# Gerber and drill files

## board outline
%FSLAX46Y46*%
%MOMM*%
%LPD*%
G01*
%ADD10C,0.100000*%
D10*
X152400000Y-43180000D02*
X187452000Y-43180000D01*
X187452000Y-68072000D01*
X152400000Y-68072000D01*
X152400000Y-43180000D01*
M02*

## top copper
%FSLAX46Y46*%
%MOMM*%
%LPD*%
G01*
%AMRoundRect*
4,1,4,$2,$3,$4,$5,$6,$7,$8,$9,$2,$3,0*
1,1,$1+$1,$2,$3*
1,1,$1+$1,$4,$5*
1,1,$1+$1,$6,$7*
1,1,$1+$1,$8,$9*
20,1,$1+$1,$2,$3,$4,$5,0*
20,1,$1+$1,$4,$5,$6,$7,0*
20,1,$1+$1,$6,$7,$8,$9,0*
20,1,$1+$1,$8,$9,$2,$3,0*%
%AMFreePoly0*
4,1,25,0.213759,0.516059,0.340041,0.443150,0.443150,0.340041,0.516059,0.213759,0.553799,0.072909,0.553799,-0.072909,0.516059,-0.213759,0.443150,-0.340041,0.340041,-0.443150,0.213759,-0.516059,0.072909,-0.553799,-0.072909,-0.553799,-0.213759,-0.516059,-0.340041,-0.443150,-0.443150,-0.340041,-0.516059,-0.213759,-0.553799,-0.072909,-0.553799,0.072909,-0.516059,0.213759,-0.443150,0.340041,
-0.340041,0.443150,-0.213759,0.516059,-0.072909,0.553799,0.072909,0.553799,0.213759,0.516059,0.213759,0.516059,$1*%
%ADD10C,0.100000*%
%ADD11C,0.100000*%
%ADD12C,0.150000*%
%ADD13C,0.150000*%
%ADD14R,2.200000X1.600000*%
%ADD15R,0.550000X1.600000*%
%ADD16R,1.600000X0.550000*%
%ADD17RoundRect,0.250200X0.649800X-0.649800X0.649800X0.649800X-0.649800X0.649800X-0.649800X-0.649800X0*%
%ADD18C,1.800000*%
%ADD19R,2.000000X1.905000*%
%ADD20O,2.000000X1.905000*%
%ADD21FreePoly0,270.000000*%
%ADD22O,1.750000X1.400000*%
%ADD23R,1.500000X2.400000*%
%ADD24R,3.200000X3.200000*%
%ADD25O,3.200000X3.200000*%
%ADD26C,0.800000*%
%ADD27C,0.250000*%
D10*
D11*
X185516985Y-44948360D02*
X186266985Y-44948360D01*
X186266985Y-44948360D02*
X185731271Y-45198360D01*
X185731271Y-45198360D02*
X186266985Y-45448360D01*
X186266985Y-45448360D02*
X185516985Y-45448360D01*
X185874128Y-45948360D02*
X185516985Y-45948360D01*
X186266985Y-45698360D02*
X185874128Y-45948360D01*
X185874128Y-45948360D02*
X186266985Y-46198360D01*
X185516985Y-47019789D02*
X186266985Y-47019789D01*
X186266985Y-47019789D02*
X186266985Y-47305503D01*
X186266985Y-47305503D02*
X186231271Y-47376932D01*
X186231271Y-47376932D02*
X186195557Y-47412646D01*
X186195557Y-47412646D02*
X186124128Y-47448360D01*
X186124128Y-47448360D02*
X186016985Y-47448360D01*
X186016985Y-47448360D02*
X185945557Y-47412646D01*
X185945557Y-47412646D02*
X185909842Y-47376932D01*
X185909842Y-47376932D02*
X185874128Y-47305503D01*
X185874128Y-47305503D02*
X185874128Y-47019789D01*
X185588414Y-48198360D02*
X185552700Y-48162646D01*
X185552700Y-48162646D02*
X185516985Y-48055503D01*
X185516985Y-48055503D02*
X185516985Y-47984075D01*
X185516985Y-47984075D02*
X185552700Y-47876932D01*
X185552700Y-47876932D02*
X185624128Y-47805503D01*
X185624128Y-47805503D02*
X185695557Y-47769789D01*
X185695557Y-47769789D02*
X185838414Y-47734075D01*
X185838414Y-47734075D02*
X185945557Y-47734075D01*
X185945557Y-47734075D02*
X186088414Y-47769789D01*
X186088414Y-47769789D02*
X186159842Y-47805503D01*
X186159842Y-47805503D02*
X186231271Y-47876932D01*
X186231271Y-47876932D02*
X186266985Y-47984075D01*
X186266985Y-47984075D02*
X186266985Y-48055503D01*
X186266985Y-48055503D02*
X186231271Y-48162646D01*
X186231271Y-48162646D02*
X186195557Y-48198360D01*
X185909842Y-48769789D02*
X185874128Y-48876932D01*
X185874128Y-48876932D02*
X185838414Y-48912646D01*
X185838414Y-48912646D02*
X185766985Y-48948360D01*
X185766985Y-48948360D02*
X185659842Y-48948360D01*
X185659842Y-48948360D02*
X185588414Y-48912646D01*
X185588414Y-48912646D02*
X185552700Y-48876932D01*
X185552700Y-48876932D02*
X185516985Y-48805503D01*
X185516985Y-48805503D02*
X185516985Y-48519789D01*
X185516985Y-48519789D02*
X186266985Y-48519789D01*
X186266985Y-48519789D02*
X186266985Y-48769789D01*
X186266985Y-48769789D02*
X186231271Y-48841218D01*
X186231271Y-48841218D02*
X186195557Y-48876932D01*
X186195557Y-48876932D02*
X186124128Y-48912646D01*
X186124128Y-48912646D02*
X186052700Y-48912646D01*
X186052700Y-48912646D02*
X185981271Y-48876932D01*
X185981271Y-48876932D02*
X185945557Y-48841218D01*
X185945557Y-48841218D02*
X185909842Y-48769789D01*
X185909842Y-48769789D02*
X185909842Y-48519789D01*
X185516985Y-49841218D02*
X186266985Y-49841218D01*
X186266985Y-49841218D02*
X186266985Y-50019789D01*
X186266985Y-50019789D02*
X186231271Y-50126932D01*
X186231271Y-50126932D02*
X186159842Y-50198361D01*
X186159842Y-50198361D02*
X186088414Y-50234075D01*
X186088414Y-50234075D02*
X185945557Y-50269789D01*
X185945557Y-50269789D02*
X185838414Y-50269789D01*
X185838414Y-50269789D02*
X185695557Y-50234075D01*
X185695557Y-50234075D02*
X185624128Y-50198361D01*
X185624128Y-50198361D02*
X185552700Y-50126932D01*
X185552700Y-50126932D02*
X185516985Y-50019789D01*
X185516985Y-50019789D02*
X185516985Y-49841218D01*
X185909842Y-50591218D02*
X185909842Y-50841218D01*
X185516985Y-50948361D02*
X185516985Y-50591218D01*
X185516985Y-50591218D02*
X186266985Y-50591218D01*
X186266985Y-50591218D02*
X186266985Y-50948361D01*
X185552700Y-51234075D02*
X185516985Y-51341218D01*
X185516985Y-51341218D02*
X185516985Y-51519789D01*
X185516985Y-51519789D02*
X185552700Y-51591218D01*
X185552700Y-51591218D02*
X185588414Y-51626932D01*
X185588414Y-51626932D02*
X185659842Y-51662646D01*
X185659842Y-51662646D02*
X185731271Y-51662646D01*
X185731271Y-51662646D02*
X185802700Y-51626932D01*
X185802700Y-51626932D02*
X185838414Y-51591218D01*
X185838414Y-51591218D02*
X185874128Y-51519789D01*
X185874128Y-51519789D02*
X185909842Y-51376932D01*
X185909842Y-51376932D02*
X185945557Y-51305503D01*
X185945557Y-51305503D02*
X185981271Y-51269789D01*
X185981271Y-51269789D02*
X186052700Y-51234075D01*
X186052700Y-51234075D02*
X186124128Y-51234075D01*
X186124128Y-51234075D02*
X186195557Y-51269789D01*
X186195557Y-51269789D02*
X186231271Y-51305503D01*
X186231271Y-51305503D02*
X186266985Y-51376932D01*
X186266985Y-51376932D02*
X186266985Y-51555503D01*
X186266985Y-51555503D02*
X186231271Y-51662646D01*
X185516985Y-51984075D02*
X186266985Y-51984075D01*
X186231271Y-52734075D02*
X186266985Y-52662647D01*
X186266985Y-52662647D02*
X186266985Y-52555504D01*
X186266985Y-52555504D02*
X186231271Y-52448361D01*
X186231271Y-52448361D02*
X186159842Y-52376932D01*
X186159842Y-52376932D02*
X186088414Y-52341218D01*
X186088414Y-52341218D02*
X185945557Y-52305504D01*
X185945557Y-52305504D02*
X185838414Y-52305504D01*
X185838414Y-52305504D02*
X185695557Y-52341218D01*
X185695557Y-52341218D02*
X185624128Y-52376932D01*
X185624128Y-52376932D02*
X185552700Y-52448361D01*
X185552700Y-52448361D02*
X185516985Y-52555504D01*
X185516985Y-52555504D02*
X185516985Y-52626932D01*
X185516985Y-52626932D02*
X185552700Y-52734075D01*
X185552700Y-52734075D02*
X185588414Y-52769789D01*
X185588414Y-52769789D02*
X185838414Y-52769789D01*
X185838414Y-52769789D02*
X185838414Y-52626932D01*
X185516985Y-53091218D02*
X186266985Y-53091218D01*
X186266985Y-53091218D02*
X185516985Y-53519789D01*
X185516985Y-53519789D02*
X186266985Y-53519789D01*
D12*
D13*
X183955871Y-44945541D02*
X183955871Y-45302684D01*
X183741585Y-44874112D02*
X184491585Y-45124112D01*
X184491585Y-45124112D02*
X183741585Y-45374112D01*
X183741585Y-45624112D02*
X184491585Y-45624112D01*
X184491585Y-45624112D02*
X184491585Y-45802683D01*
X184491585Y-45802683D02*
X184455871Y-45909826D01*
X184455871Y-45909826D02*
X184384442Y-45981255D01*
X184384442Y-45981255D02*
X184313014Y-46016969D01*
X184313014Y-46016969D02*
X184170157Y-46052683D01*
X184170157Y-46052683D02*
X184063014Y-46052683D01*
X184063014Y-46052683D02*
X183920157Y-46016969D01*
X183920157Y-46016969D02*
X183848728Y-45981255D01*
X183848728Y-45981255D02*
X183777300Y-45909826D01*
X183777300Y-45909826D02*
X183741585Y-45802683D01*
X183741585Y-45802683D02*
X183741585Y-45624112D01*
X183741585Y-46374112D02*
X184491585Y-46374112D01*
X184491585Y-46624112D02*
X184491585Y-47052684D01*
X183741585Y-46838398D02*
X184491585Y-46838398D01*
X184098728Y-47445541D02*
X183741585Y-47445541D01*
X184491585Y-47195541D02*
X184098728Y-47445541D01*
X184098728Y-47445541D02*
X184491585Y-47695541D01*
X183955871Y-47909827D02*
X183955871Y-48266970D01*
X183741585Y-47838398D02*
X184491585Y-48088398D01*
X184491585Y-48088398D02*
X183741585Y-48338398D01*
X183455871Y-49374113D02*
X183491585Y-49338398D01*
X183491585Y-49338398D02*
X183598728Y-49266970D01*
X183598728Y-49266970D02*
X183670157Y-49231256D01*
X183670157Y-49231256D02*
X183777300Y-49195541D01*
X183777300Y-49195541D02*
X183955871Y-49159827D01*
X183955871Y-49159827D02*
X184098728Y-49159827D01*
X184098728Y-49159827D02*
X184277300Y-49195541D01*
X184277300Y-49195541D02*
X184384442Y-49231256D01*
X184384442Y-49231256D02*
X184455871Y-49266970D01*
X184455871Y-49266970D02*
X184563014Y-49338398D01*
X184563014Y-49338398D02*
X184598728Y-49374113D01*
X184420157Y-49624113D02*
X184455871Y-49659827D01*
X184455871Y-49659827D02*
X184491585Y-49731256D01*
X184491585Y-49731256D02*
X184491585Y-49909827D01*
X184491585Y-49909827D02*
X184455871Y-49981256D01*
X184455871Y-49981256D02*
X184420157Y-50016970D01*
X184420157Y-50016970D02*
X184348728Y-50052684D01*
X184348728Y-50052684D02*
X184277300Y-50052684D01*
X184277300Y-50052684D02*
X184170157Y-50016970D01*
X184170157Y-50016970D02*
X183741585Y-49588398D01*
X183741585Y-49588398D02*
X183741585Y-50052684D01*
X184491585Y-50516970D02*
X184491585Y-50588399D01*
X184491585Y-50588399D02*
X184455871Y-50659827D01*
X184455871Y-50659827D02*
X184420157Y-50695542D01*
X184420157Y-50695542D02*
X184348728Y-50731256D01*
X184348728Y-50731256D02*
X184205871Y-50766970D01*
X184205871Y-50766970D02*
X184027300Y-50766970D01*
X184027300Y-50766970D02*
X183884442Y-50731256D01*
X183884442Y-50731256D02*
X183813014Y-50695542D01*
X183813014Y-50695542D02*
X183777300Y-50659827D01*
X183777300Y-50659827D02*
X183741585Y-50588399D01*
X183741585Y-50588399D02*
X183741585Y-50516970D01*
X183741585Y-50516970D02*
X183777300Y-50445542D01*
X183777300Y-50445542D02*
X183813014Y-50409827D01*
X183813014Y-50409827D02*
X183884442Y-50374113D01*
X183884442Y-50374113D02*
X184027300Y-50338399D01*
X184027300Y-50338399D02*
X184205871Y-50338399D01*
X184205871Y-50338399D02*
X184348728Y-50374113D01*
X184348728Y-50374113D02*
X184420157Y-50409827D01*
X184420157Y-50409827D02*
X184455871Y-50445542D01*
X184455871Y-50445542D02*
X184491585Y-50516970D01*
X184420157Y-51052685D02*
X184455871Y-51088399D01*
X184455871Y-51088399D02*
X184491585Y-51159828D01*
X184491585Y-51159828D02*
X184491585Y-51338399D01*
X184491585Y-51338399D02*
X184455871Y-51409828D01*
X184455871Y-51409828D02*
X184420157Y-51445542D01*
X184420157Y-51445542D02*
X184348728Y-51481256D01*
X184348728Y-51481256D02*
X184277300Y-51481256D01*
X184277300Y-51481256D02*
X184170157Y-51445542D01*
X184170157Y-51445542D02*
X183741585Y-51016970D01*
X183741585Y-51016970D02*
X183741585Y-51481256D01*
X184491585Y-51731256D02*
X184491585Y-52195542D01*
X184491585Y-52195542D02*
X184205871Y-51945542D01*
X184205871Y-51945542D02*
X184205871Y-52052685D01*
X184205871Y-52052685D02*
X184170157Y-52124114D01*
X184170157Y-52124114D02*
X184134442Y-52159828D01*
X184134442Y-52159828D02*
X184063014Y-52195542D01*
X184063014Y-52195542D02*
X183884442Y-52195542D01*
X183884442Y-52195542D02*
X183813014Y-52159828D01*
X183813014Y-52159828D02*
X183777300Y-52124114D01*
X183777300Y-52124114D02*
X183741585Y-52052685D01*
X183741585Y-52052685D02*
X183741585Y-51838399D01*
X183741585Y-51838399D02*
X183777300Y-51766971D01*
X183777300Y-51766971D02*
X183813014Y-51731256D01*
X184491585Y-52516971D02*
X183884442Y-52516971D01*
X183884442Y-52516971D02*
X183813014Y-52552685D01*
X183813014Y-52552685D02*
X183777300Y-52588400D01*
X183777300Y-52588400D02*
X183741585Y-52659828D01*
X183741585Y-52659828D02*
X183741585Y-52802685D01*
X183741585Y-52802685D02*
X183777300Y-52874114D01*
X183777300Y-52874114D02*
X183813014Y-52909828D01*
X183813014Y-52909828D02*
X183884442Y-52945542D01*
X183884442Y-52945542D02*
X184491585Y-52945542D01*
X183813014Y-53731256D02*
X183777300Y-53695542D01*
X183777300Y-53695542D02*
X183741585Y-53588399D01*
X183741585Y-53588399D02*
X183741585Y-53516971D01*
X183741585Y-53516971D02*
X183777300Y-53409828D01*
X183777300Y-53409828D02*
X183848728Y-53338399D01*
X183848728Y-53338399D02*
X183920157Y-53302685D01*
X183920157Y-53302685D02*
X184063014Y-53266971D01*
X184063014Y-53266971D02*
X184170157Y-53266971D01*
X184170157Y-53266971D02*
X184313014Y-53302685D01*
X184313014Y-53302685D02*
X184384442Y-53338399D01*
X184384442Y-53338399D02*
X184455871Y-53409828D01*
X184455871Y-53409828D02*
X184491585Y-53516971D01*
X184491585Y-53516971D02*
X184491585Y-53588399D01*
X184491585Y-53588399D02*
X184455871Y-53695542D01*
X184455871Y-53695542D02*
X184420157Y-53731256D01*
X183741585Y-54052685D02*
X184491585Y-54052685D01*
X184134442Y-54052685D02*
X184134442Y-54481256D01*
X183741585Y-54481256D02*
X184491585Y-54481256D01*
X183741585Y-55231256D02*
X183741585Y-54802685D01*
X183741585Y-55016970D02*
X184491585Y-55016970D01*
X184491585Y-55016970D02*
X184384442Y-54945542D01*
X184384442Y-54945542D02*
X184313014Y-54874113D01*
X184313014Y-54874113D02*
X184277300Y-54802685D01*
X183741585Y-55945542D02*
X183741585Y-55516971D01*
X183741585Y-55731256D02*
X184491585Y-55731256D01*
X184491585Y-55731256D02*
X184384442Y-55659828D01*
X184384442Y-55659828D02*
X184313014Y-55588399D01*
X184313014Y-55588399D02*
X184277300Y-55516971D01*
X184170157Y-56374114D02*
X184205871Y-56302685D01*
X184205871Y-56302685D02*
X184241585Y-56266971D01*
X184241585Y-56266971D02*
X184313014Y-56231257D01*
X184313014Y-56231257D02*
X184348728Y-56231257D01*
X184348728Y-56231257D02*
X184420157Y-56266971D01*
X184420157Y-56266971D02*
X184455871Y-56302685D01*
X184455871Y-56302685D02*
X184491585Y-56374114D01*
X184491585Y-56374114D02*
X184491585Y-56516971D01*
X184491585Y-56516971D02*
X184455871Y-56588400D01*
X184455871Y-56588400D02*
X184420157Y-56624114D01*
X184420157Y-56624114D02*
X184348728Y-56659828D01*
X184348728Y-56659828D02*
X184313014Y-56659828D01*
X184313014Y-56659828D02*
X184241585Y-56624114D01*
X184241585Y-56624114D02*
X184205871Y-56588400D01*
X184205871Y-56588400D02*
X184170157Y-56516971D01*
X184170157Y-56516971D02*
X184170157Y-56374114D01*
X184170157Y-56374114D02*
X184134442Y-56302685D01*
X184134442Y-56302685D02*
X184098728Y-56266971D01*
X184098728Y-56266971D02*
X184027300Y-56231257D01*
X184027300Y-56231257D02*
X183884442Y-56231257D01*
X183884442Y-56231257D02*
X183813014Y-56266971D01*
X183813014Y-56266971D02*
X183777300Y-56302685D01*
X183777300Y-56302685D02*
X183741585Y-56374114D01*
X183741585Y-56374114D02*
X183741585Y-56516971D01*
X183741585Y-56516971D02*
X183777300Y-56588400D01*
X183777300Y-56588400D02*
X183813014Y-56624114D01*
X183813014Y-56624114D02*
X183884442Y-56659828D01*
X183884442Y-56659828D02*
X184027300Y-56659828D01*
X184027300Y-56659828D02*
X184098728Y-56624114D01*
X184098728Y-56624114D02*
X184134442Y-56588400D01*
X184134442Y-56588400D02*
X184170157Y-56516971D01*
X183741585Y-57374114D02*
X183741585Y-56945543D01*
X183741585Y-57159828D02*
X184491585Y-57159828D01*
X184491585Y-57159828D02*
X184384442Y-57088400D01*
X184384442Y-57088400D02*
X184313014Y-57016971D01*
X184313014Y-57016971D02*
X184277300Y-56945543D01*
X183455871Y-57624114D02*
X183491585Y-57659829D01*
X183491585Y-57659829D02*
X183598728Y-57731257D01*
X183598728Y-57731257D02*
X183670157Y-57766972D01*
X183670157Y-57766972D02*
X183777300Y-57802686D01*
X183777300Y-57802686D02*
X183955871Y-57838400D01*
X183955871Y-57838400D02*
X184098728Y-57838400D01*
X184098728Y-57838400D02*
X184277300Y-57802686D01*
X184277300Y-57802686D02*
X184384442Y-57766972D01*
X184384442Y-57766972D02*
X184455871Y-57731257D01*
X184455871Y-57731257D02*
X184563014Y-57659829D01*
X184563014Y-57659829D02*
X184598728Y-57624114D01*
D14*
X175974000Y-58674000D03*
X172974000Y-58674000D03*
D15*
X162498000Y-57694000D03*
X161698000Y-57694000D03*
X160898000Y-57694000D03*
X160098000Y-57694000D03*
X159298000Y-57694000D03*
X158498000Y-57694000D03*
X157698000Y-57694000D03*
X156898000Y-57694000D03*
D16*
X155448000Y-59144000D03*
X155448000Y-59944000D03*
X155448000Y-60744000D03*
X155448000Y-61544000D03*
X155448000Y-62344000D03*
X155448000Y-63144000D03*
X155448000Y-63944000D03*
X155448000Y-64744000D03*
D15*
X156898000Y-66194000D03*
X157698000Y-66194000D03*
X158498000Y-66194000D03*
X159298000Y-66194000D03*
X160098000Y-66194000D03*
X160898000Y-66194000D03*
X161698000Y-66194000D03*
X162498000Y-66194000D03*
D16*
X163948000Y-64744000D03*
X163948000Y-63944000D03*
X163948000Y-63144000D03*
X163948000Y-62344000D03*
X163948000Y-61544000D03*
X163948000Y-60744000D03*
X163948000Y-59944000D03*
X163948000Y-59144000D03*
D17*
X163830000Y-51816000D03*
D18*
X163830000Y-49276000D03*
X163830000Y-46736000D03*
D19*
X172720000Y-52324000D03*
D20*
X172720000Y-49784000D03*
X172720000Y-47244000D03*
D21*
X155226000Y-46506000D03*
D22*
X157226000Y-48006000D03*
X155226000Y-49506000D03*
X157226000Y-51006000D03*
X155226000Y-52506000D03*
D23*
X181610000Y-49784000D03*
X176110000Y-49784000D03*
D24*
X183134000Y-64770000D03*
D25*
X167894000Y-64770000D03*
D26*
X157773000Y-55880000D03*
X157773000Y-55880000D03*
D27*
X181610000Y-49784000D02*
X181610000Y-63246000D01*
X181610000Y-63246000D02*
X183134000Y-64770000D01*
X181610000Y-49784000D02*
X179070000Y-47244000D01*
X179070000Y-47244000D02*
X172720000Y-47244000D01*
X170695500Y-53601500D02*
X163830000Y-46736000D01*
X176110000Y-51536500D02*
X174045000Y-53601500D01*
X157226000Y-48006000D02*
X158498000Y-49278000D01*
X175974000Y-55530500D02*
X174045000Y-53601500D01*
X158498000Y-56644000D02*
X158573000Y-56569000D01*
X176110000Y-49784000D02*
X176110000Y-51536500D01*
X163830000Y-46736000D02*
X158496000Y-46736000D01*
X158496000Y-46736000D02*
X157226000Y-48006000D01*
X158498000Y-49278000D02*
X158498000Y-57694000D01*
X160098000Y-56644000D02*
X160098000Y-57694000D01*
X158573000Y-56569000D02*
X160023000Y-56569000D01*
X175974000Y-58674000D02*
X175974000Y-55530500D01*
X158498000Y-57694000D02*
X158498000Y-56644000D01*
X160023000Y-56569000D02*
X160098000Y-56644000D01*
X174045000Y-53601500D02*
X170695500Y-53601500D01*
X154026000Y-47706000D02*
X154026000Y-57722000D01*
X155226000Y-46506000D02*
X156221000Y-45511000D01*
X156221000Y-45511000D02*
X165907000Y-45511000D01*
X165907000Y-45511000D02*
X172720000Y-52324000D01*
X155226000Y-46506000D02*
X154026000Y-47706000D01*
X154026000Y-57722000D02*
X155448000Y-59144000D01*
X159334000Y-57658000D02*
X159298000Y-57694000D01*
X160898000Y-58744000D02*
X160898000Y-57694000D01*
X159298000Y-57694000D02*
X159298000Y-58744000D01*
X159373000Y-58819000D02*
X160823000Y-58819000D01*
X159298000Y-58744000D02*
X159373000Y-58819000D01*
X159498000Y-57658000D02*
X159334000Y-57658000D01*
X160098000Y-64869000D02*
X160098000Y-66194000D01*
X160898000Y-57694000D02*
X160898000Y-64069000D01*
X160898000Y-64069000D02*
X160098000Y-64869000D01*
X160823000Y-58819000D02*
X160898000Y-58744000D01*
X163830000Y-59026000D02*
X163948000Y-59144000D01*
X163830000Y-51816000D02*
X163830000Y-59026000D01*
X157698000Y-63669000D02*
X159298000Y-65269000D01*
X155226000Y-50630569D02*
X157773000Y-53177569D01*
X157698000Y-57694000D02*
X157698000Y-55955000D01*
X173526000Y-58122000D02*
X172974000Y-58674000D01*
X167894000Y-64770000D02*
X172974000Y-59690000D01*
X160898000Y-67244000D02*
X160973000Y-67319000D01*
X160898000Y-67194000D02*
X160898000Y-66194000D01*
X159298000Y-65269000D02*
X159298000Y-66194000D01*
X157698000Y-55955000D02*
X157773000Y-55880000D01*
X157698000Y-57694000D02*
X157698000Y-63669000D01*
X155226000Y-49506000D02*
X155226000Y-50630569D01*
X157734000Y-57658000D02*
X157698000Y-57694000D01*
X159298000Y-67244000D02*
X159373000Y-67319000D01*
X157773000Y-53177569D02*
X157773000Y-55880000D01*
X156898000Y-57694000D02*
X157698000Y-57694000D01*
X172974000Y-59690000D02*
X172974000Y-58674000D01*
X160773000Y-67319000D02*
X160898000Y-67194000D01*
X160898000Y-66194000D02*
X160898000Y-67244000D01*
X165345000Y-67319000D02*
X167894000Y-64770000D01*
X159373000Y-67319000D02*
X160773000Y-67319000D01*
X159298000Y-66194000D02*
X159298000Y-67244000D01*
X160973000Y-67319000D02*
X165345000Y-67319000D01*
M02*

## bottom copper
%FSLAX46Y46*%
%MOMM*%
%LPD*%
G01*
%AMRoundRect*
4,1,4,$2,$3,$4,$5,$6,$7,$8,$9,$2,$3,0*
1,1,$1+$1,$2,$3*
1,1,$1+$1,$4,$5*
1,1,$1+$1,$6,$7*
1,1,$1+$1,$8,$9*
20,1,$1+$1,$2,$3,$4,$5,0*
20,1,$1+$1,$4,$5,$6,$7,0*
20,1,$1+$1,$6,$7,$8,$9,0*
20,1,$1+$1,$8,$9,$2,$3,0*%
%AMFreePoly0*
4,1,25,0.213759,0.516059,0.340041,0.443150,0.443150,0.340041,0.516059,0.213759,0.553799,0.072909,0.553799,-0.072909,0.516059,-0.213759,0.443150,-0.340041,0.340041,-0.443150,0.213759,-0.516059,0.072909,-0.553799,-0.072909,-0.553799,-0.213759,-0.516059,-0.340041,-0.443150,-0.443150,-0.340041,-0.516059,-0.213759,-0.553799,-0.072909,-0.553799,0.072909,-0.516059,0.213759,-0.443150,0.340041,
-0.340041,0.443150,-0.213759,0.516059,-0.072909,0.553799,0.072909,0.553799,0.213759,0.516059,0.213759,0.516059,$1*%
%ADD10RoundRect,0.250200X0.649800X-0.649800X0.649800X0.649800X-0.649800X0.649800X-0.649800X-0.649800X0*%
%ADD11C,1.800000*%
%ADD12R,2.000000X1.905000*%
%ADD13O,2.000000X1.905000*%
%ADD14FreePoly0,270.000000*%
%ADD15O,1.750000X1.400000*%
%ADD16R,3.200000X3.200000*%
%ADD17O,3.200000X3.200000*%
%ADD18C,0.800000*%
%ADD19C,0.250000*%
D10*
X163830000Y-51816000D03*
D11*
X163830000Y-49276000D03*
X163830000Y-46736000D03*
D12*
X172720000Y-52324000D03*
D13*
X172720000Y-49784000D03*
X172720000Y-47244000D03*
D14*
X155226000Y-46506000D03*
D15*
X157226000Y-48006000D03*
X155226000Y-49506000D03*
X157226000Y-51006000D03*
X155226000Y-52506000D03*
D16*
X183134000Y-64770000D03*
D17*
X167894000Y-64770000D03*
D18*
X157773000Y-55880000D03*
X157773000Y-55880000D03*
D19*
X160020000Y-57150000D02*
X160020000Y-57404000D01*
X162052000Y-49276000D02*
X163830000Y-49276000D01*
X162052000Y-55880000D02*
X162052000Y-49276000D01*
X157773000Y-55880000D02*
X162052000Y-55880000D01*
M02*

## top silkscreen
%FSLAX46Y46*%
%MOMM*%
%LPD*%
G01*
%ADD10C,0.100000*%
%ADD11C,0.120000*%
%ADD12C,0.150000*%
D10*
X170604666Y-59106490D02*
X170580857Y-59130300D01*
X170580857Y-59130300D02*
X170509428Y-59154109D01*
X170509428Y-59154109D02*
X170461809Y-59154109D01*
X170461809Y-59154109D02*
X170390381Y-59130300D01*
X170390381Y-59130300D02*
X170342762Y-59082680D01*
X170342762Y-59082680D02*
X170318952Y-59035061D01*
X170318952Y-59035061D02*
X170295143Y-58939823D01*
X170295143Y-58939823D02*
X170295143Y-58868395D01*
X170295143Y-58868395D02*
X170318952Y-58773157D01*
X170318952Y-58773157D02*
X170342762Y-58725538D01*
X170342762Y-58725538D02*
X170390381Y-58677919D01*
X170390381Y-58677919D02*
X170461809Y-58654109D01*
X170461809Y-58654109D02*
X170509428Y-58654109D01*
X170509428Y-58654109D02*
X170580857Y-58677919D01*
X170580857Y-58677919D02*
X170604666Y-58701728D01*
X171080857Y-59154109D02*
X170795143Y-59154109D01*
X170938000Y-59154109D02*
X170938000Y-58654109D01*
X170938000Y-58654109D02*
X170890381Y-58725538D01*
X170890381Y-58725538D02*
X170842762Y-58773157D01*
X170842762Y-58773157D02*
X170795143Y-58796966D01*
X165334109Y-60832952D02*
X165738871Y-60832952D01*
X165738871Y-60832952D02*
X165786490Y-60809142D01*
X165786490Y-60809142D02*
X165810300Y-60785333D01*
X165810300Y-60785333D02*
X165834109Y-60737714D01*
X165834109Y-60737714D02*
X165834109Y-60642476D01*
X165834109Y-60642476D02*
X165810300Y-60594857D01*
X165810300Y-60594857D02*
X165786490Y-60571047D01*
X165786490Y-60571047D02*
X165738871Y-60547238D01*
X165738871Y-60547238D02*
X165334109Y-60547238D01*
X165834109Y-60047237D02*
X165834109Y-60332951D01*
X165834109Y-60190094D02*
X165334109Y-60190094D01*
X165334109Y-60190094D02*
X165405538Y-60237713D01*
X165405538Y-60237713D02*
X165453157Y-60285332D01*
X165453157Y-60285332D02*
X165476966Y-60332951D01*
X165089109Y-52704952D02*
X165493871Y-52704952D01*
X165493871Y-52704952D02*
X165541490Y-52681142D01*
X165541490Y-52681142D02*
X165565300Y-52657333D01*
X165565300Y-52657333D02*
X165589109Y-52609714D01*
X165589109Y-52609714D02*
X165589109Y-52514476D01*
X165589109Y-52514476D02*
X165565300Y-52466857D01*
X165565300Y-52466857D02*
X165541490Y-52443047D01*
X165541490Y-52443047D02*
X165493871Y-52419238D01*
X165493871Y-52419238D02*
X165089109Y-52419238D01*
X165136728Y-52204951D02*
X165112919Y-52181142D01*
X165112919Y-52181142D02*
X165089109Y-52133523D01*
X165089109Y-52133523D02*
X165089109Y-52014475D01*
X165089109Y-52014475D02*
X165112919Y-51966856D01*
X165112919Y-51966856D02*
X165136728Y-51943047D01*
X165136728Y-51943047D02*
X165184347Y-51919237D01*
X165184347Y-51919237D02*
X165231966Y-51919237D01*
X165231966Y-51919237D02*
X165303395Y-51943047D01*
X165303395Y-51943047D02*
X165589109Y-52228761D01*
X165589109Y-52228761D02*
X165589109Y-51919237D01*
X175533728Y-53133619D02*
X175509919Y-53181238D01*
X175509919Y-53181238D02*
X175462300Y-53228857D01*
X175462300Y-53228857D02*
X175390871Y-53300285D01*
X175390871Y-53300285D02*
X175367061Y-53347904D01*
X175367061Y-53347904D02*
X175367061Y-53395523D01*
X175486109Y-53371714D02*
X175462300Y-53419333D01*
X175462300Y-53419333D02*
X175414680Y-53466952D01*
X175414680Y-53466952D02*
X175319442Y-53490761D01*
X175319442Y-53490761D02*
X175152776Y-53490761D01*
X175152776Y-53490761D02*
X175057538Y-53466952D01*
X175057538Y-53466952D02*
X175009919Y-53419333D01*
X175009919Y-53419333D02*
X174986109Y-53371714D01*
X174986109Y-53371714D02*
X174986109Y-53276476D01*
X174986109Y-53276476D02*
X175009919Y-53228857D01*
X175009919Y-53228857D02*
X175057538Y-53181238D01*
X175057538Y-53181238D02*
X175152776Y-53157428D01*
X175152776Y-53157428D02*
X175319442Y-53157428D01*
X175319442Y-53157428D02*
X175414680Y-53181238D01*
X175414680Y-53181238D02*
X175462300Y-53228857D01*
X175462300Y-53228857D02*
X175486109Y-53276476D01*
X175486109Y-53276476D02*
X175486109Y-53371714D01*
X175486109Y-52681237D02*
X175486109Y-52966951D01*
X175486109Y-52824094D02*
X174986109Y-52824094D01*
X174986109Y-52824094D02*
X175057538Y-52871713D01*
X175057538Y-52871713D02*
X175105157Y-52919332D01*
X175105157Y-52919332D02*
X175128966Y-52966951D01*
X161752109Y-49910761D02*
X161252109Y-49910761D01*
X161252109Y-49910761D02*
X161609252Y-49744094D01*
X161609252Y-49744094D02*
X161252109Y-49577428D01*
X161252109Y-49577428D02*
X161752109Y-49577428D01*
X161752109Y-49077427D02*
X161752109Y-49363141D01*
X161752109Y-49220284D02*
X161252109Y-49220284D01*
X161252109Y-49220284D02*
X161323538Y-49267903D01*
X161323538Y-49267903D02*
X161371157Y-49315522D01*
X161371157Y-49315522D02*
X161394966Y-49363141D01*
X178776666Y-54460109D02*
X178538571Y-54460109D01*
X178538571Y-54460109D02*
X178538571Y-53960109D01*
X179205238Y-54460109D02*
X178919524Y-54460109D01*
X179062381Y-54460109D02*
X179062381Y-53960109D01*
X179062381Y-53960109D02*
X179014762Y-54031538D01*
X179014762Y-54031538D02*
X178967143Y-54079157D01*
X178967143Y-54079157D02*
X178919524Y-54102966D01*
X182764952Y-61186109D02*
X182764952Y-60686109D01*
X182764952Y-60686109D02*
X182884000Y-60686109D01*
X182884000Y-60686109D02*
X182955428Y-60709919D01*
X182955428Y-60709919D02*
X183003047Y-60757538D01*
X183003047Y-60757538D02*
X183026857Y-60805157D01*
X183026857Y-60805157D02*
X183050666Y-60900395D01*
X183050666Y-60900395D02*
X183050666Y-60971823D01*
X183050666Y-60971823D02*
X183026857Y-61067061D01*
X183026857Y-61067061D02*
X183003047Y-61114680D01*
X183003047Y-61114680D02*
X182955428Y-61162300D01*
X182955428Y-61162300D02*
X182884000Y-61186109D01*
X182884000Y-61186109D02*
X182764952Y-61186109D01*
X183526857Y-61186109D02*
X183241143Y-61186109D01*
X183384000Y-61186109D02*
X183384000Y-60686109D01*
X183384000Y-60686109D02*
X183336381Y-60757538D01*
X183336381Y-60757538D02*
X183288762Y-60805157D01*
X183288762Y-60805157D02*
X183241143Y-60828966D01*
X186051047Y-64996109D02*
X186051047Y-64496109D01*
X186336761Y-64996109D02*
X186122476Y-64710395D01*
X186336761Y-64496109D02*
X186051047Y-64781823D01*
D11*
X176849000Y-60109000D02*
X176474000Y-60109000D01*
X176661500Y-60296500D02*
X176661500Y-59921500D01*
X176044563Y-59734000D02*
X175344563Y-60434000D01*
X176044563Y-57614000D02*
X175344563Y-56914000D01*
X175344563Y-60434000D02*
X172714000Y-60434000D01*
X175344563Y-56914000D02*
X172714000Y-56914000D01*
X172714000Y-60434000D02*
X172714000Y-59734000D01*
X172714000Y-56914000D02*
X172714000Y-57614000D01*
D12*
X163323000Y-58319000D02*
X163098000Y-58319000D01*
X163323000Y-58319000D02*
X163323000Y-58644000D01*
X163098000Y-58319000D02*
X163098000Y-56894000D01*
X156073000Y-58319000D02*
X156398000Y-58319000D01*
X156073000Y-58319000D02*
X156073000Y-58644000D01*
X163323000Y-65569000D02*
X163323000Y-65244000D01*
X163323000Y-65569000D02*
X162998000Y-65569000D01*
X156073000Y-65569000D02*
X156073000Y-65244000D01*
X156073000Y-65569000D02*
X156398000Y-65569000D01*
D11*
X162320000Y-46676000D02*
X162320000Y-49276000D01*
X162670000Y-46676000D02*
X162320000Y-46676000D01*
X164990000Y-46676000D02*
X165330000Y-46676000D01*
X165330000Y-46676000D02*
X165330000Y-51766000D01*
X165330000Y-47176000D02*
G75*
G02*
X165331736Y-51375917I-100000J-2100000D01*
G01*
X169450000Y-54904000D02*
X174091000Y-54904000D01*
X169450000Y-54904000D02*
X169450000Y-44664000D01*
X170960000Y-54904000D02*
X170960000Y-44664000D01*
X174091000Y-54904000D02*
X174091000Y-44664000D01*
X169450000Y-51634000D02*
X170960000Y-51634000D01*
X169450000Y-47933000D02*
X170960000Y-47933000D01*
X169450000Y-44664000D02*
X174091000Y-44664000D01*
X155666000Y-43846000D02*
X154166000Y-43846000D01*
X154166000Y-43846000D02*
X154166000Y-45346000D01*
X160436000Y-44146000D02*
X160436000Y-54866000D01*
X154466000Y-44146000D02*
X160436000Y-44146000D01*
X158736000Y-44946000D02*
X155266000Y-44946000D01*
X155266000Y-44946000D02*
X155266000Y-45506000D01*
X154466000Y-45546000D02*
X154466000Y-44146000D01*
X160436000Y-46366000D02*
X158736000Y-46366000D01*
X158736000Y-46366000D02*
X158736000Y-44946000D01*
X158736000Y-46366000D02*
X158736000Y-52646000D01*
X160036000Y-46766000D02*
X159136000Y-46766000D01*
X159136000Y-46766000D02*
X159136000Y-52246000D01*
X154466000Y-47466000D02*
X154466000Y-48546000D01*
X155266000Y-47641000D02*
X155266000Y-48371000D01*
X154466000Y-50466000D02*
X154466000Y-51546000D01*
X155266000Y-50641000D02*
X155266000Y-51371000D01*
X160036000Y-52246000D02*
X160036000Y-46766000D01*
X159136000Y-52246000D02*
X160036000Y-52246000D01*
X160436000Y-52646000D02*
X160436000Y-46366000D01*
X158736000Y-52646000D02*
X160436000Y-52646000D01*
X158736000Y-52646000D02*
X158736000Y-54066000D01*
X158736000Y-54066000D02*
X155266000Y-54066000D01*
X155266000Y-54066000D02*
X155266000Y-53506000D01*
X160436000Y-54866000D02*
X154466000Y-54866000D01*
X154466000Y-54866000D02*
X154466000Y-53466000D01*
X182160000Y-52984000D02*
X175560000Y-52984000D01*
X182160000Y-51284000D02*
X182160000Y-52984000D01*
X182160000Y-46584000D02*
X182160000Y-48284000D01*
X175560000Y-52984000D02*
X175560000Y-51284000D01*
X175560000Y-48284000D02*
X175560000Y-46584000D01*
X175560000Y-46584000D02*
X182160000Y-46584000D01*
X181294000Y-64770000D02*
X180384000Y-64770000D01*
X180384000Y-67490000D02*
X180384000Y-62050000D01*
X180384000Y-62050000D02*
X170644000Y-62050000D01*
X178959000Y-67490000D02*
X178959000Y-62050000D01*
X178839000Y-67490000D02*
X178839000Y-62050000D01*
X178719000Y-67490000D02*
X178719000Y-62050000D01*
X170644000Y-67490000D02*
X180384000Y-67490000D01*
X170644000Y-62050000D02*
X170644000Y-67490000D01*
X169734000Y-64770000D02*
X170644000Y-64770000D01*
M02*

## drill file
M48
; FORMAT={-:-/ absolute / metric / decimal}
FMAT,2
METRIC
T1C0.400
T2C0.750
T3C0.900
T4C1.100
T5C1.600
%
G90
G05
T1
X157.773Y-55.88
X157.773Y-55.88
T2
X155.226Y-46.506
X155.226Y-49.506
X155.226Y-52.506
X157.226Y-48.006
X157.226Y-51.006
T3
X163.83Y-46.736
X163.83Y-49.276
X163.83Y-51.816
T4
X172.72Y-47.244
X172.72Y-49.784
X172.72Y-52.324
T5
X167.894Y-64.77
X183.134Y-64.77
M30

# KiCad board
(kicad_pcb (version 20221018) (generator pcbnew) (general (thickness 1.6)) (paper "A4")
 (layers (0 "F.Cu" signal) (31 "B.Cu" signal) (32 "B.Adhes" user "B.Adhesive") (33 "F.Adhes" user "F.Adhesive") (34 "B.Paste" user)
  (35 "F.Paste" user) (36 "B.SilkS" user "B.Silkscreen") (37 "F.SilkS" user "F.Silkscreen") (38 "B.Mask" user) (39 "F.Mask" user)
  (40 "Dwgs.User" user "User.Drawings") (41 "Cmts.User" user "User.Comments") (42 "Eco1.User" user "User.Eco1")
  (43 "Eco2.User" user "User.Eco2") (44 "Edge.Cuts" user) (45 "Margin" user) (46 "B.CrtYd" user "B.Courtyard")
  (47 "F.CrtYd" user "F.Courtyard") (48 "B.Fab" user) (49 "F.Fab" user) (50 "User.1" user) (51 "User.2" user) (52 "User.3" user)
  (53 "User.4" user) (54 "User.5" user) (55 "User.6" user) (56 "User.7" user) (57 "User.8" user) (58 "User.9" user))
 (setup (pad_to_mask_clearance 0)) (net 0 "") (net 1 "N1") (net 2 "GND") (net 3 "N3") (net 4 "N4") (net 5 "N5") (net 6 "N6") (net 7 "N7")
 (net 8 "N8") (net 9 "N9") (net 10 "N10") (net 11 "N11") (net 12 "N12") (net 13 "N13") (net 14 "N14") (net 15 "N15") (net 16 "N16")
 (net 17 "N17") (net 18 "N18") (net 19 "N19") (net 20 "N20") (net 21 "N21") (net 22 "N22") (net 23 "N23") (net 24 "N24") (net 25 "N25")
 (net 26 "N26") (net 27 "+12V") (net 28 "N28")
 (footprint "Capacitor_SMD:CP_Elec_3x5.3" (layer "F.Cu") (at 174.474 58.674 180)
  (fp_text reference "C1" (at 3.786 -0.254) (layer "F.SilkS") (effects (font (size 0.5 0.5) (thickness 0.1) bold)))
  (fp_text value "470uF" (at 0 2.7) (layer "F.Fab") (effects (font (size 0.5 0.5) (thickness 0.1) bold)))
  (fp_line (start -2.375 -1.435) (end -2 -1.435) (stroke (width 0.12) (type solid)) (layer "F.SilkS"))
  (fp_line (start -2.1875 -1.6225) (end -2.1875 -1.2475) (stroke (width 0.12) (type solid)) (layer "F.SilkS"))
  (fp_line (start -1.570563 -1.06) (end -0.870563 -1.76) (stroke (width 0.12) (type solid)) (layer "F.SilkS"))
  (fp_line (start -1.570563 1.06) (end -0.870563 1.76) (stroke (width 0.12) (type solid)) (layer "F.SilkS"))
  (fp_line (start -0.870563 -1.76) (end 1.76 -1.76) (stroke (width 0.12) (type solid)) (layer "F.SilkS"))
  (fp_line (start -0.870563 1.76) (end 1.76 1.76) (stroke (width 0.12) (type solid)) (layer "F.SilkS"))
  (fp_line (start 1.76 -1.76) (end 1.76 -1.06) (stroke (width 0.12) (type solid)) (layer "F.SilkS"))
  (fp_line (start 1.76 1.76) (end 1.76 1.06) (stroke (width 0.12) (type solid)) (layer "F.SilkS"))
  (pad "1" smd rect (at -1.5 0 180) (size 2.2 1.6) (layers "F.Cu" "F.Paste" "F.Mask") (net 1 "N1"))
  (pad "2" smd rect (at 1.5 0 180) (size 2.2 1.6) (layers "F.Cu" "F.Paste" "F.Mask") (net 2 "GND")))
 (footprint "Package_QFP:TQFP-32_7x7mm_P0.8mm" (layer "F.Cu") (at 159.698 61.944 -90)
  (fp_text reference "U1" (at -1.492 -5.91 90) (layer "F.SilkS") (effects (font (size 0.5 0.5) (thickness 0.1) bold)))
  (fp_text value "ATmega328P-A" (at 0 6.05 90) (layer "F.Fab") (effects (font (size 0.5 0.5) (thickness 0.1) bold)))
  (fp_line (start -3.625 -3.625) (end -3.625 -3.4) (stroke (width 0.15) (type solid)) (layer "F.SilkS"))
  (fp_line (start -3.625 -3.625) (end -3.3 -3.625) (stroke (width 0.15) (type solid)) (layer "F.SilkS"))
  (fp_line (start -3.625 -3.4) (end -5.05 -3.4) (stroke (width 0.15) (type solid)) (layer "F.SilkS"))
  (fp_line (start -3.625 3.625) (end -3.625 3.3) (stroke (width 0.15) (type solid)) (layer "F.SilkS"))
  (fp_line (start -3.625 3.625) (end -3.3 3.625) (stroke (width 0.15) (type solid)) (layer "F.SilkS"))
  (fp_line (start 3.625 -3.625) (end 3.3 -3.625) (stroke (width 0.15) (type solid)) (layer "F.SilkS"))
  (fp_line (start 3.625 -3.625) (end 3.625 -3.3) (stroke (width 0.15) (type solid)) (layer "F.SilkS"))
  (fp_line (start 3.625 3.625) (end 3.3 3.625) (stroke (width 0.15) (type solid)) (layer "F.SilkS"))
  (fp_line (start 3.625 3.625) (end 3.625 3.3) (stroke (width 0.15) (type solid)) (layer "F.SilkS"))
  (pad "1" smd rect (at -4.25 -2.8 270) (size 1.6 0.55) (layers "F.Cu" "F.Paste" "F.Mask") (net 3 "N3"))
  (pad "2" smd rect (at -4.25 -2 270) (size 1.6 0.55) (layers "F.Cu" "F.Paste" "F.Mask") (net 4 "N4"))
  (pad "3" smd rect (at -4.25 -1.2 270) (size 1.6 0.55) (layers "F.Cu" "F.Paste" "F.Mask") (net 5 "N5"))
  (pad "4" smd rect (at -4.25 -0.4 270) (size 1.6 0.55) (layers "F.Cu" "F.Paste" "F.Mask") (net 1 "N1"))
  (pad "5" smd rect (at -4.25 0.4 270) (size 1.6 0.55) (layers "F.Cu" "F.Paste" "F.Mask") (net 5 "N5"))
  (pad "6" smd rect (at -4.25 1.2 270) (size 1.6 0.55) (layers "F.Cu" "F.Paste" "F.Mask") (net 1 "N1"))
  (pad "7" smd rect (at -4.25 2 270) (size 1.6 0.55) (layers "F.Cu" "F.Paste" "F.Mask") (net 2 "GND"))
  (pad "8" smd rect (at -4.25 2.8 270) (size 1.6 0.55) (layers "F.Cu" "F.Paste" "F.Mask") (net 2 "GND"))
  (pad "9" smd rect (at -2.8 4.25) (size 1.6 0.55) (layers "F.Cu" "F.Paste" "F.Mask") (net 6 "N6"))
  (pad "10" smd rect (at -2 4.25) (size 1.6 0.55) (layers "F.Cu" "F.Paste" "F.Mask") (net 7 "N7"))
  (pad "11" smd rect (at -1.2 4.25) (size 1.6 0.55) (layers "F.Cu" "F.Paste" "F.Mask") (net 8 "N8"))
  (pad "12" smd rect (at -0.4 4.25) (size 1.6 0.55) (layers "F.Cu" "F.Paste" "F.Mask") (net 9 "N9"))
  (pad "13" smd rect (at 0.4 4.25) (size 1.6 0.55) (layers "F.Cu" "F.Paste" "F.Mask") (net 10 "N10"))
  (pad "14" smd rect (at 1.2 4.25) (size 1.6 0.55) (layers "F.Cu" "F.Paste" "F.Mask") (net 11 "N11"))
  (pad "15" smd rect (at 2 4.25) (size 1.6 0.55) (layers "F.Cu" "F.Paste" "F.Mask") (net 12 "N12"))
  (pad "16" smd rect (at 2.8 4.25) (size 1.6 0.55) (layers "F.Cu" "F.Paste" "F.Mask") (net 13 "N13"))
  (pad "17" smd rect (at 4.25 2.8 270) (size 1.6 0.55) (layers "F.Cu" "F.Paste" "F.Mask") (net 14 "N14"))
  (pad "18" smd rect (at 4.25 2 270) (size 1.6 0.55) (layers "F.Cu" "F.Paste" "F.Mask") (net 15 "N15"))
  (pad "19" smd rect (at 4.25 1.2 270) (size 1.6 0.55) (layers "F.Cu" "F.Paste" "F.Mask") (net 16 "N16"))
  (pad "20" smd rect (at 4.25 0.4 270) (size 1.6 0.55) (layers "F.Cu" "F.Paste" "F.Mask") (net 2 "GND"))
  (pad "21" smd rect (at 4.25 -0.4 270) (size 1.6 0.55) (layers "F.Cu" "F.Paste" "F.Mask") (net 5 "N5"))
  (pad "22" smd rect (at 4.25 -1.2 270) (size 1.6 0.55) (layers "F.Cu" "F.Paste" "F.Mask") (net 2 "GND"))
  (pad "23" smd rect (at 4.25 -2 270) (size 1.6 0.55) (layers "F.Cu" "F.Paste" "F.Mask") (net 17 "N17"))
  (pad "24" smd rect (at 4.25 -2.8 270) (size 1.6 0.55) (layers "F.Cu" "F.Paste" "F.Mask") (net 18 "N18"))
  (pad "25" smd rect (at 2.8 -4.25) (size 1.6 0.55) (layers "F.Cu" "F.Paste" "F.Mask") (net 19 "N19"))
  (pad "26" smd rect (at 2 -4.25) (size 1.6 0.55) (layers "F.Cu" "F.Paste" "F.Mask") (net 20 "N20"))
  (pad "27" smd rect (at 1.2 -4.25) (size 1.6 0.55) (layers "F.Cu" "F.Paste" "F.Mask") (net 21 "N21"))
  (pad "28" smd rect (at 0.4 -4.25) (size 1.6 0.55) (layers "F.Cu" "F.Paste" "F.Mask") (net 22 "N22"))
  (pad "29" smd rect (at -0.4 -4.25) (size 1.6 0.55) (layers "F.Cu" "F.Paste" "F.Mask") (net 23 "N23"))
  (pad "30" smd rect (at -1.2 -4.25) (size 1.6 0.55) (layers "F.Cu" "F.Paste" "F.Mask") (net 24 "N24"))
  (pad "31" smd rect (at -2 -4.25) (size 1.6 0.55) (layers "F.Cu" "F.Paste" "F.Mask") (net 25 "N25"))
  (pad "32" smd rect (at -2.8 -4.25) (size 1.6 0.55) (layers "F.Cu" "F.Paste" "F.Mask") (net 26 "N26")))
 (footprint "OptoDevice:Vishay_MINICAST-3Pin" (layer "F.Cu") (at 163.83 51.816 90)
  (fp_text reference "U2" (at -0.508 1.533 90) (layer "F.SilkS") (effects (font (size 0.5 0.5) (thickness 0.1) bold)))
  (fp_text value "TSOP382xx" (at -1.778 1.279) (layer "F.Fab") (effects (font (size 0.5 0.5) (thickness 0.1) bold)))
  (fp_line (start 5.14 -1.51) (end 2.54 -1.51) (stroke (width 0.12) (type solid)) (layer "F.SilkS"))
  (fp_line (start 5.14 -1.16) (end 5.14 -1.51) (stroke (width 0.12) (type solid)) (layer "F.SilkS"))
  (fp_line (start 5.14 1.16) (end 5.14 1.5) (stroke (width 0.12) (type solid)) (layer "F.SilkS"))
  (fp_line (start 5.14 1.5) (end 0.05 1.5) (stroke (width 0.12) (type solid)) (layer "F.SilkS"))
  (fp_arc (start 4.64 1.5) (mid 2.540869 3.502379) (end 0.440083 1.501736) (stroke (width 0.12) (type solid)) (layer "F.SilkS"))
  (pad "1" thru_hole roundrect (at 0 0 90) (size 1.8 1.8) (drill 0.9) (layers "*.Cu" "*.Mask") (roundrect_rratio 0.139) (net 26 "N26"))
  (pad "2" thru_hole circle (at 2.54 0 90) (size 1.8 1.8) (drill 0.9) (layers "*.Cu" "*.Mask") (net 2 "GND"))
  (pad "3" thru_hole circle (at 5.08 0 90) (size 1.8 1.8) (drill 0.9) (layers "*.Cu" "*.Mask") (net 1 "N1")))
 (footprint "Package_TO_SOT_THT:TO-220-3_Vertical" (layer "F.Cu") (at 172.72 52.324 90)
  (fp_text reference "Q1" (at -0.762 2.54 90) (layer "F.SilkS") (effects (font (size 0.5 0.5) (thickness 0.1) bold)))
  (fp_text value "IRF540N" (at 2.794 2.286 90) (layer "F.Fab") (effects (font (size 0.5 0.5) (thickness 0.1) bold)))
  (fp_line (start -2.58 -3.27) (end -2.58 1.371) (stroke (width 0.12) (type solid)) (layer "F.SilkS"))
  (fp_line (start -2.58 -3.27) (end 7.66 -3.27) (stroke (width 0.12) (type solid)) (layer "F.SilkS"))
  (fp_line (start -2.58 -1.76) (end 7.66 -1.76) (stroke (width 0.12) (type solid)) (layer "F.SilkS"))
  (fp_line (start -2.58 1.371) (end 7.66 1.371) (stroke (width 0.12) (type solid)) (layer "F.SilkS"))
  (fp_line (start 0.69 -3.27) (end 0.69 -1.76) (stroke (width 0.12) (type solid)) (layer "F.SilkS"))
  (fp_line (start 4.391 -3.27) (end 4.391 -1.76) (stroke (width 0.12) (type solid)) (layer "F.SilkS"))
  (fp_line (start 7.66 -3.27) (end 7.66 1.371) (stroke (width 0.12) (type solid)) (layer "F.SilkS"))
  (pad "1" thru_hole rect (at 0 0 90) (size 1.905 2) (drill 1.1) (layers "*.Cu" "*.Mask") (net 6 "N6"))
  (pad "2" thru_hole oval (at 2.54 0 90) (size 1.905 2) (drill 1.1) (layers "*.Cu" "*.Mask") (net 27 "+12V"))
  (pad "3" thru_hole oval (at 5.08 0 90) (size 1.905 2) (drill 1.1) (layers "*.Cu" "*.Mask") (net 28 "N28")))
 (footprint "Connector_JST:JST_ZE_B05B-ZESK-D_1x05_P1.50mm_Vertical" (layer "F.Cu") (at 155.226 46.506 -90)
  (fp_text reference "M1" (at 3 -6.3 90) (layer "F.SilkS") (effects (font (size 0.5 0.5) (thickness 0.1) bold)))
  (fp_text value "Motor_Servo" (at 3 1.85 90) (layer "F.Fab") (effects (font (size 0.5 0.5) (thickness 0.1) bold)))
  (fp_line (start -2.66 -0.44) (end -2.66 1.06) (stroke (width 0.12) (type solid)) (layer "F.SilkS"))
  (fp_line (start -2.66 1.06) (end -1.16 1.06) (stroke (width 0.12) (type solid)) (layer "F.SilkS"))
  (fp_line (start -2.36 -5.21) (end 8.36 -5.21) (stroke (width 0.12) (type solid)) (layer "F.SilkS"))
  (fp_line (start -2.36 0.76) (end -2.36 -5.21) (stroke (width 0.12) (type solid)) (layer "F.SilkS"))
  (fp_line (start -1.56 -3.51) (end -1.56 -0.04) (stroke (width 0.12) (type solid)) (layer "F.SilkS"))
  (fp_line (start -1.56 -0.04) (end -1 -0.04) (stroke (width 0.12) (type solid)) (layer "F.SilkS"))
  (fp_line (start -0.96 0.76) (end -2.36 0.76) (stroke (width 0.12) (type solid)) (layer "F.SilkS"))
  (fp_line (start -0.14 -5.21) (end -0.14 -3.51) (stroke (width 0.12) (type solid)) (layer "F.SilkS"))
  (fp_line (start -0.14 -3.51) (end -1.56 -3.51) (stroke (width 0.12) (type solid)) (layer "F.SilkS"))
  (fp_line (start -0.14 -3.51) (end 6.14 -3.51) (stroke (width 0.12) (type solid)) (layer "F.SilkS"))
  (fp_line (start 0.26 -4.81) (end 0.26 -3.91) (stroke (width 0.12) (type solid)) (layer "F.SilkS"))
  (fp_line (start 0.26 -3.91) (end 5.74 -3.91) (stroke (width 0.12) (type solid)) (layer "F.SilkS"))
  (fp_line (start 0.96 0.76) (end 2.04 0.76) (stroke (width 0.12) (type solid)) (layer "F.SilkS"))
  (fp_line (start 1.135 -0.04) (end 1.865 -0.04) (stroke (width 0.12) (type solid)) (layer "F.SilkS"))
  (fp_line (start 3.96 0.76) (end 5.04 0.76) (stroke (width 0.12) (type solid)) (layer "F.SilkS"))
  (fp_line (start 4.135 -0.04) (end 4.865 -0.04) (stroke (width 0.12) (type solid)) (layer "F.SilkS"))
  (fp_line (start 5.74 -4.81) (end 0.26 -4.81) (stroke (width 0.12) (type solid)) (layer "F.SilkS"))
  (fp_line (start 5.74 -3.91) (end 5.74 -4.81) (stroke (width 0.12) (type solid)) (layer "F.SilkS"))
  (fp_line (start 6.14 -5.21) (end -0.14 -5.21) (stroke (width 0.12) (type solid)) (layer "F.SilkS"))
  (fp_line (start 6.14 -3.51) (end 6.14 -5.21) (stroke (width 0.12) (type solid)) (layer "F.SilkS"))
  (fp_line (start 6.14 -3.51) (end 7.56 -3.51) (stroke (width 0.12) (type solid)) (layer "F.SilkS"))
  (fp_line (start 7.56 -3.51) (end 7.56 -0.04) (stroke (width 0.12) (type solid)) (layer "F.SilkS"))
  (fp_line (start 7.56 -0.04) (end 7 -0.04) (stroke (width 0.12) (type solid)) (layer "F.SilkS"))
  (fp_line (start 8.36 -5.21) (end 8.36 0.76) (stroke (width 0.12) (type solid)) (layer "F.SilkS"))
  (fp_line (start 8.36 0.76) (end 6.96 0.76) (stroke (width 0.12) (type solid)) (layer "F.SilkS"))
  (pad "1" thru_hole custom (at 0 0 270) (size 1.117157 1.117157) (drill 0.75) (layers "*.Cu" "*.Mask") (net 6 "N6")
   (thermal_bridge_angle 90) (options (clearance outline) (anchor circle)) (primitives))
  (pad "2" thru_hole oval (at 1.5 -2 270) (size 1.4 1.75) (drill 0.75) (layers "*.Cu" "*.Mask") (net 1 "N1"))
  (pad "3" thru_hole oval (at 3 0 270) (size 1.4 1.75) (drill 0.75) (layers "*.Cu" "*.Mask") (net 2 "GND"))
  (pad "4" thru_hole oval (at 4.5 -2 270) (size 1.4 1.75) (drill 0.75) (layers "*.Cu" "*.Mask"))
  (pad "5" thru_hole oval (at 6 0 270) (size 1.4 1.75) (drill 0.75) (layers "*.Cu" "*.Mask")))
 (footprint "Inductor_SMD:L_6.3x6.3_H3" (layer "F.Cu") (at 178.86 49.784 180)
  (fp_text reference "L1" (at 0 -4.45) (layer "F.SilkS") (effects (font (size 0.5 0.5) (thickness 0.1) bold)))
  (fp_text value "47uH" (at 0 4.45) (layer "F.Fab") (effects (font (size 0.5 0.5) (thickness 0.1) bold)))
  (fp_line (start -3.3 -3.2) (end 3.3 -3.2) (stroke (width 0.12) (type solid)) (layer "F.SilkS"))
  (fp_line (start -3.3 -1.5) (end -3.3 -3.2) (stroke (width 0.12) (type solid)) (layer "F.SilkS"))
  (fp_line (start -3.3 3.2) (end -3.3 1.5) (stroke (width 0.12) (type solid)) (layer "F.SilkS"))
  (fp_line (start 3.3 -3.2) (end 3.3 -1.5) (stroke (width 0.12) (type solid)) (layer "F.SilkS"))
  (fp_line (start 3.3 1.5) (end 3.3 3.2) (stroke (width 0.12) (type solid)) (layer "F.SilkS"))
  (fp_line (start 3.3 3.2) (end -3.3 3.2) (stroke (width 0.12) (type solid)) (layer "F.SilkS"))
  (pad "1" smd rect (at -2.75 0 180) (size 1.5 2.4) (layers "F.Cu" "F.Paste" "F.Mask") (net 28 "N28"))
  (pad "2" smd rect (at 2.75 0 180) (size 1.5 2.4) (layers "F.Cu" "F.Paste" "F.Mask") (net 1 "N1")))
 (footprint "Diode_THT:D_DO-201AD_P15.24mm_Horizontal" (layer "F.Cu") (at 183.134 64.77 180)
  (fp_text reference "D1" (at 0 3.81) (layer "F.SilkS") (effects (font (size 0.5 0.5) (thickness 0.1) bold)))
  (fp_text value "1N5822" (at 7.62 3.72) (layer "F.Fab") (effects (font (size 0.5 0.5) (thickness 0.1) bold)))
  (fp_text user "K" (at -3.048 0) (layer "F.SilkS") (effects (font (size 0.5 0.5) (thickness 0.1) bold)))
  (fp_line (start 1.84 0) (end 2.75 0) (stroke (width 0.12) (type solid)) (layer "F.SilkS"))
  (fp_line (start 2.75 -2.72) (end 2.75 2.72) (stroke (width 0.12) (type solid)) (layer "F.SilkS"))
  (fp_line (start 2.75 2.72) (end 12.49 2.72) (stroke (width 0.12) (type solid)) (layer "F.SilkS"))
  (fp_line (start 4.175 -2.72) (end 4.175 2.72) (stroke (width 0.12) (type solid)) (layer "F.SilkS"))
  (fp_line (start 4.295 -2.72) (end 4.295 2.72) (stroke (width 0.12) (type solid)) (layer "F.SilkS"))
  (fp_line (start 4.415 -2.72) (end 4.415 2.72) (stroke (width 0.12) (type solid)) (layer "F.SilkS"))
  (fp_line (start 12.49 -2.72) (end 2.75 -2.72) (stroke (width 0.12) (type solid)) (layer "F.SilkS"))
  (fp_line (start 12.49 2.72) (end 12.49 -2.72) (stroke (width 0.12) (type solid)) (layer "F.SilkS"))
  (fp_line (start 13.4 0) (end 12.49 0) (stroke (width 0.12) (type solid)) (layer "F.SilkS"))
  (pad "1" thru_hole rect (at 0 0 180) (size 3.2 3.2) (drill 1.6) (layers "*.Cu" "*.Mask") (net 28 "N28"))
  (pad "2" thru_hole oval (at 15.24 0 180) (size 3.2 3.2) (drill 1.6) (layers "*.Cu" "*.Mask") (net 2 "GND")))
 (gr_rect (start 152.4 43.18) (end 187.452 68.072) (stroke (width 0.1) (type default)) (fill none) (layer "Edge.Cuts"))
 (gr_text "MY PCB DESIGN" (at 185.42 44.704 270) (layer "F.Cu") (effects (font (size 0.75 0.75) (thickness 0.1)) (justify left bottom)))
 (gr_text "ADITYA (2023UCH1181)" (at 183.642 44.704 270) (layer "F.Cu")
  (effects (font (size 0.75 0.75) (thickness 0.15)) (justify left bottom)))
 (segment (start 181.61 49.784) (end 181.61 63.246) (width 0.25) (layer "F.Cu") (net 28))
 (segment (start 181.61 63.246) (end 183.134 64.77) (width 0.25) (layer "F.Cu") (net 28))
 (segment (start 181.61 49.784) (end 179.07 47.244) (width 0.25) (layer "F.Cu") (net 28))
 (segment (start 179.07 47.244) (end 172.72 47.244) (width 0.25) (layer "F.Cu") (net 28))
 (segment (start 170.6955 53.6015) (end 163.83 46.736) (width 0.25) (layer "F.Cu") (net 1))
 (segment (start 176.11 51.5365) (end 174.045 53.6015) (width 0.25) (layer "F.Cu") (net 1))
 (segment (start 157.226 48.006) (end 158.498 49.278) (width 0.25) (layer "F.Cu") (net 1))
 (segment (start 175.974 55.5305) (end 174.045 53.6015) (width 0.25) (layer "F.Cu") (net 1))
 (segment (start 158.498 56.644) (end 158.573 56.569) (width 0.25) (layer "F.Cu") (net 1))
 (segment (start 176.11 49.784) (end 176.11 51.5365) (width 0.25) (layer "F.Cu") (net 1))
 (segment (start 163.83 46.736) (end 158.496 46.736) (width 0.25) (layer "F.Cu") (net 1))
 (segment (start 158.496 46.736) (end 157.226 48.006) (width 0.25) (layer "F.Cu") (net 1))
 (segment (start 158.498 49.278) (end 158.498 57.694) (width 0.25) (layer "F.Cu") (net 1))
 (segment (start 160.098 56.644) (end 160.098 57.694) (width 0.25) (layer "F.Cu") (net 1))
 (segment (start 158.573 56.569) (end 160.023 56.569) (width 0.25) (layer "F.Cu") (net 1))
 (segment (start 175.974 58.674) (end 175.974 55.5305) (width 0.25) (layer "F.Cu") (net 1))
 (segment (start 158.498 57.694) (end 158.498 56.644) (width 0.25) (layer "F.Cu") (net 1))
 (segment (start 160.023 56.569) (end 160.098 56.644) (width 0.25) (layer "F.Cu") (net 1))
 (segment (start 174.045 53.6015) (end 170.6955 53.6015) (width 0.25) (layer "F.Cu") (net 1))
 (segment (start 160.02 57.15) (end 160.02 57.404) (width 0.25) (layer "B.Cu") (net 1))
 (segment (start 154.026 47.706) (end 154.026 57.722) (width 0.25) (layer "F.Cu") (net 6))
 (segment (start 155.226 46.506) (end 156.221 45.511) (width 0.25) (layer "F.Cu") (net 6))
 (segment (start 156.221 45.511) (end 165.907 45.511) (width 0.25) (layer "F.Cu") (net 6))
 (segment (start 165.907 45.511) (end 172.72 52.324) (width 0.25) (layer "F.Cu") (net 6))
 (segment (start 155.226 46.506) (end 154.026 47.706) (width 0.25) (layer "F.Cu") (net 6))
 (segment (start 154.026 57.722) (end 155.448 59.144) (width 0.25) (layer "F.Cu") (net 6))
 (segment (start 159.334 57.658) (end 159.298 57.694) (width 0.25) (layer "F.Cu") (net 5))
 (segment (start 160.898 58.744) (end 160.898 57.694) (width 0.25) (layer "F.Cu") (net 5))
 (segment (start 159.298 57.694) (end 159.298 58.744) (width 0.25) (layer "F.Cu") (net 5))
 (segment (start 159.373 58.819) (end 160.823 58.819) (width 0.25) (layer "F.Cu") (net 5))
 (segment (start 159.298 58.744) (end 159.373 58.819) (width 0.25) (layer "F.Cu") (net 5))
 (segment (start 159.498 57.658) (end 159.334 57.658) (width 0.25) (layer "F.Cu") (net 5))
 (segment (start 160.098 64.869) (end 160.098 66.194) (width 0.25) (layer "F.Cu") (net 5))
 (segment (start 160.898 57.694) (end 160.898 64.069) (width 0.25) (layer "F.Cu") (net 5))
 (segment (start 160.898 64.069) (end 160.098 64.869) (width 0.25) (layer "F.Cu") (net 5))
 (segment (start 160.823 58.819) (end 160.898 58.744) (width 0.25) (layer "F.Cu") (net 5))
 (segment (start 163.83 59.026) (end 163.948 59.144) (width 0.25) (layer "F.Cu") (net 26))
 (segment (start 163.83 51.816) (end 163.83 59.026) (width 0.25) (layer "F.Cu") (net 26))
 (segment (start 157.698 63.669) (end 159.298 65.269) (width 0.25) (layer "F.Cu") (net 2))
 (segment (start 155.226 50.630569) (end 157.773 53.177569) (width 0.25) (layer "F.Cu") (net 2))
 (segment (start 157.698 57.694) (end 157.698 55.955) (width 0.25) (layer "F.Cu") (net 2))
 (segment (start 173.526 58.122) (end 172.974 58.674) (width 0.25) (layer "F.Cu") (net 2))
 (segment (start 167.894 64.77) (end 172.974 59.69) (width 0.25) (layer "F.Cu") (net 2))
 (segment (start 160.898 67.244) (end 160.973 67.319) (width 0.25) (layer "F.Cu") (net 2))
 (segment (start 160.898 67.194) (end 160.898 66.194) (width 0.25) (layer "F.Cu") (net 2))
 (segment (start 159.298 65.269) (end 159.298 66.194) (width 0.25) (layer "F.Cu") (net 2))
 (segment (start 157.698 55.955) (end 157.773 55.88) (width 0.25) (layer "F.Cu") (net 2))
 (segment (start 157.698 57.694) (end 157.698 63.669) (width 0.25) (layer "F.Cu") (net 2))
 (segment (start 155.226 49.506) (end 155.226 50.630569) (width 0.25) (layer "F.Cu") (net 2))
 (segment (start 157.734 57.658) (end 157.698 57.694) (width 0.25) (layer "F.Cu") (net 2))
 (segment (start 159.298 67.244) (end 159.373 67.319) (width 0.25) (layer "F.Cu") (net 2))
 (segment (start 157.773 53.177569) (end 157.773 55.88) (width 0.25) (layer "F.Cu") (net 2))
 (segment (start 156.898 57.694) (end 157.698 57.694) (width 0.25) (layer "F.Cu") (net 2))
 (segment (start 172.974 59.69) (end 172.974 58.674) (width 0.25) (layer "F.Cu") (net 2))
 (segment (start 160.773 67.319) (end 160.898 67.194) (width 0.25) (layer "F.Cu") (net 2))
 (segment (start 160.898 66.194) (end 160.898 67.244) (width 0.25) (layer "F.Cu") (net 2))
 (segment (start 165.345 67.319) (end 167.894 64.77) (width 0.25) (layer "F.Cu") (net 2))
 (segment (start 159.373 67.319) (end 160.773 67.319) (width 0.25) (layer "F.Cu") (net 2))
 (segment (start 159.298 66.194) (end 159.298 67.244) (width 0.25) (layer "F.Cu") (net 2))
 (segment (start 160.973 67.319) (end 165.345 67.319) (width 0.25) (layer "F.Cu") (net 2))
 (via (at 157.773 55.88) (size 0.8) (drill 0.4) (layers "F.Cu" "B.Cu") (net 2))
 (via (at 157.773 55.88) (size 0.8) (drill 0.4) (layers "F.Cu" "B.Cu") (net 2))
 (segment (start 162.052 49.276) (end 163.83 49.276) (width 0.25) (layer "B.Cu") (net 2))
 (segment (start 162.052 55.88) (end 162.052 49.276) (width 0.25) (layer "B.Cu") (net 2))
 (segment (start 157.773 55.88) (end 162.052 55.88) (width 0.25) (layer "B.Cu") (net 2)))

